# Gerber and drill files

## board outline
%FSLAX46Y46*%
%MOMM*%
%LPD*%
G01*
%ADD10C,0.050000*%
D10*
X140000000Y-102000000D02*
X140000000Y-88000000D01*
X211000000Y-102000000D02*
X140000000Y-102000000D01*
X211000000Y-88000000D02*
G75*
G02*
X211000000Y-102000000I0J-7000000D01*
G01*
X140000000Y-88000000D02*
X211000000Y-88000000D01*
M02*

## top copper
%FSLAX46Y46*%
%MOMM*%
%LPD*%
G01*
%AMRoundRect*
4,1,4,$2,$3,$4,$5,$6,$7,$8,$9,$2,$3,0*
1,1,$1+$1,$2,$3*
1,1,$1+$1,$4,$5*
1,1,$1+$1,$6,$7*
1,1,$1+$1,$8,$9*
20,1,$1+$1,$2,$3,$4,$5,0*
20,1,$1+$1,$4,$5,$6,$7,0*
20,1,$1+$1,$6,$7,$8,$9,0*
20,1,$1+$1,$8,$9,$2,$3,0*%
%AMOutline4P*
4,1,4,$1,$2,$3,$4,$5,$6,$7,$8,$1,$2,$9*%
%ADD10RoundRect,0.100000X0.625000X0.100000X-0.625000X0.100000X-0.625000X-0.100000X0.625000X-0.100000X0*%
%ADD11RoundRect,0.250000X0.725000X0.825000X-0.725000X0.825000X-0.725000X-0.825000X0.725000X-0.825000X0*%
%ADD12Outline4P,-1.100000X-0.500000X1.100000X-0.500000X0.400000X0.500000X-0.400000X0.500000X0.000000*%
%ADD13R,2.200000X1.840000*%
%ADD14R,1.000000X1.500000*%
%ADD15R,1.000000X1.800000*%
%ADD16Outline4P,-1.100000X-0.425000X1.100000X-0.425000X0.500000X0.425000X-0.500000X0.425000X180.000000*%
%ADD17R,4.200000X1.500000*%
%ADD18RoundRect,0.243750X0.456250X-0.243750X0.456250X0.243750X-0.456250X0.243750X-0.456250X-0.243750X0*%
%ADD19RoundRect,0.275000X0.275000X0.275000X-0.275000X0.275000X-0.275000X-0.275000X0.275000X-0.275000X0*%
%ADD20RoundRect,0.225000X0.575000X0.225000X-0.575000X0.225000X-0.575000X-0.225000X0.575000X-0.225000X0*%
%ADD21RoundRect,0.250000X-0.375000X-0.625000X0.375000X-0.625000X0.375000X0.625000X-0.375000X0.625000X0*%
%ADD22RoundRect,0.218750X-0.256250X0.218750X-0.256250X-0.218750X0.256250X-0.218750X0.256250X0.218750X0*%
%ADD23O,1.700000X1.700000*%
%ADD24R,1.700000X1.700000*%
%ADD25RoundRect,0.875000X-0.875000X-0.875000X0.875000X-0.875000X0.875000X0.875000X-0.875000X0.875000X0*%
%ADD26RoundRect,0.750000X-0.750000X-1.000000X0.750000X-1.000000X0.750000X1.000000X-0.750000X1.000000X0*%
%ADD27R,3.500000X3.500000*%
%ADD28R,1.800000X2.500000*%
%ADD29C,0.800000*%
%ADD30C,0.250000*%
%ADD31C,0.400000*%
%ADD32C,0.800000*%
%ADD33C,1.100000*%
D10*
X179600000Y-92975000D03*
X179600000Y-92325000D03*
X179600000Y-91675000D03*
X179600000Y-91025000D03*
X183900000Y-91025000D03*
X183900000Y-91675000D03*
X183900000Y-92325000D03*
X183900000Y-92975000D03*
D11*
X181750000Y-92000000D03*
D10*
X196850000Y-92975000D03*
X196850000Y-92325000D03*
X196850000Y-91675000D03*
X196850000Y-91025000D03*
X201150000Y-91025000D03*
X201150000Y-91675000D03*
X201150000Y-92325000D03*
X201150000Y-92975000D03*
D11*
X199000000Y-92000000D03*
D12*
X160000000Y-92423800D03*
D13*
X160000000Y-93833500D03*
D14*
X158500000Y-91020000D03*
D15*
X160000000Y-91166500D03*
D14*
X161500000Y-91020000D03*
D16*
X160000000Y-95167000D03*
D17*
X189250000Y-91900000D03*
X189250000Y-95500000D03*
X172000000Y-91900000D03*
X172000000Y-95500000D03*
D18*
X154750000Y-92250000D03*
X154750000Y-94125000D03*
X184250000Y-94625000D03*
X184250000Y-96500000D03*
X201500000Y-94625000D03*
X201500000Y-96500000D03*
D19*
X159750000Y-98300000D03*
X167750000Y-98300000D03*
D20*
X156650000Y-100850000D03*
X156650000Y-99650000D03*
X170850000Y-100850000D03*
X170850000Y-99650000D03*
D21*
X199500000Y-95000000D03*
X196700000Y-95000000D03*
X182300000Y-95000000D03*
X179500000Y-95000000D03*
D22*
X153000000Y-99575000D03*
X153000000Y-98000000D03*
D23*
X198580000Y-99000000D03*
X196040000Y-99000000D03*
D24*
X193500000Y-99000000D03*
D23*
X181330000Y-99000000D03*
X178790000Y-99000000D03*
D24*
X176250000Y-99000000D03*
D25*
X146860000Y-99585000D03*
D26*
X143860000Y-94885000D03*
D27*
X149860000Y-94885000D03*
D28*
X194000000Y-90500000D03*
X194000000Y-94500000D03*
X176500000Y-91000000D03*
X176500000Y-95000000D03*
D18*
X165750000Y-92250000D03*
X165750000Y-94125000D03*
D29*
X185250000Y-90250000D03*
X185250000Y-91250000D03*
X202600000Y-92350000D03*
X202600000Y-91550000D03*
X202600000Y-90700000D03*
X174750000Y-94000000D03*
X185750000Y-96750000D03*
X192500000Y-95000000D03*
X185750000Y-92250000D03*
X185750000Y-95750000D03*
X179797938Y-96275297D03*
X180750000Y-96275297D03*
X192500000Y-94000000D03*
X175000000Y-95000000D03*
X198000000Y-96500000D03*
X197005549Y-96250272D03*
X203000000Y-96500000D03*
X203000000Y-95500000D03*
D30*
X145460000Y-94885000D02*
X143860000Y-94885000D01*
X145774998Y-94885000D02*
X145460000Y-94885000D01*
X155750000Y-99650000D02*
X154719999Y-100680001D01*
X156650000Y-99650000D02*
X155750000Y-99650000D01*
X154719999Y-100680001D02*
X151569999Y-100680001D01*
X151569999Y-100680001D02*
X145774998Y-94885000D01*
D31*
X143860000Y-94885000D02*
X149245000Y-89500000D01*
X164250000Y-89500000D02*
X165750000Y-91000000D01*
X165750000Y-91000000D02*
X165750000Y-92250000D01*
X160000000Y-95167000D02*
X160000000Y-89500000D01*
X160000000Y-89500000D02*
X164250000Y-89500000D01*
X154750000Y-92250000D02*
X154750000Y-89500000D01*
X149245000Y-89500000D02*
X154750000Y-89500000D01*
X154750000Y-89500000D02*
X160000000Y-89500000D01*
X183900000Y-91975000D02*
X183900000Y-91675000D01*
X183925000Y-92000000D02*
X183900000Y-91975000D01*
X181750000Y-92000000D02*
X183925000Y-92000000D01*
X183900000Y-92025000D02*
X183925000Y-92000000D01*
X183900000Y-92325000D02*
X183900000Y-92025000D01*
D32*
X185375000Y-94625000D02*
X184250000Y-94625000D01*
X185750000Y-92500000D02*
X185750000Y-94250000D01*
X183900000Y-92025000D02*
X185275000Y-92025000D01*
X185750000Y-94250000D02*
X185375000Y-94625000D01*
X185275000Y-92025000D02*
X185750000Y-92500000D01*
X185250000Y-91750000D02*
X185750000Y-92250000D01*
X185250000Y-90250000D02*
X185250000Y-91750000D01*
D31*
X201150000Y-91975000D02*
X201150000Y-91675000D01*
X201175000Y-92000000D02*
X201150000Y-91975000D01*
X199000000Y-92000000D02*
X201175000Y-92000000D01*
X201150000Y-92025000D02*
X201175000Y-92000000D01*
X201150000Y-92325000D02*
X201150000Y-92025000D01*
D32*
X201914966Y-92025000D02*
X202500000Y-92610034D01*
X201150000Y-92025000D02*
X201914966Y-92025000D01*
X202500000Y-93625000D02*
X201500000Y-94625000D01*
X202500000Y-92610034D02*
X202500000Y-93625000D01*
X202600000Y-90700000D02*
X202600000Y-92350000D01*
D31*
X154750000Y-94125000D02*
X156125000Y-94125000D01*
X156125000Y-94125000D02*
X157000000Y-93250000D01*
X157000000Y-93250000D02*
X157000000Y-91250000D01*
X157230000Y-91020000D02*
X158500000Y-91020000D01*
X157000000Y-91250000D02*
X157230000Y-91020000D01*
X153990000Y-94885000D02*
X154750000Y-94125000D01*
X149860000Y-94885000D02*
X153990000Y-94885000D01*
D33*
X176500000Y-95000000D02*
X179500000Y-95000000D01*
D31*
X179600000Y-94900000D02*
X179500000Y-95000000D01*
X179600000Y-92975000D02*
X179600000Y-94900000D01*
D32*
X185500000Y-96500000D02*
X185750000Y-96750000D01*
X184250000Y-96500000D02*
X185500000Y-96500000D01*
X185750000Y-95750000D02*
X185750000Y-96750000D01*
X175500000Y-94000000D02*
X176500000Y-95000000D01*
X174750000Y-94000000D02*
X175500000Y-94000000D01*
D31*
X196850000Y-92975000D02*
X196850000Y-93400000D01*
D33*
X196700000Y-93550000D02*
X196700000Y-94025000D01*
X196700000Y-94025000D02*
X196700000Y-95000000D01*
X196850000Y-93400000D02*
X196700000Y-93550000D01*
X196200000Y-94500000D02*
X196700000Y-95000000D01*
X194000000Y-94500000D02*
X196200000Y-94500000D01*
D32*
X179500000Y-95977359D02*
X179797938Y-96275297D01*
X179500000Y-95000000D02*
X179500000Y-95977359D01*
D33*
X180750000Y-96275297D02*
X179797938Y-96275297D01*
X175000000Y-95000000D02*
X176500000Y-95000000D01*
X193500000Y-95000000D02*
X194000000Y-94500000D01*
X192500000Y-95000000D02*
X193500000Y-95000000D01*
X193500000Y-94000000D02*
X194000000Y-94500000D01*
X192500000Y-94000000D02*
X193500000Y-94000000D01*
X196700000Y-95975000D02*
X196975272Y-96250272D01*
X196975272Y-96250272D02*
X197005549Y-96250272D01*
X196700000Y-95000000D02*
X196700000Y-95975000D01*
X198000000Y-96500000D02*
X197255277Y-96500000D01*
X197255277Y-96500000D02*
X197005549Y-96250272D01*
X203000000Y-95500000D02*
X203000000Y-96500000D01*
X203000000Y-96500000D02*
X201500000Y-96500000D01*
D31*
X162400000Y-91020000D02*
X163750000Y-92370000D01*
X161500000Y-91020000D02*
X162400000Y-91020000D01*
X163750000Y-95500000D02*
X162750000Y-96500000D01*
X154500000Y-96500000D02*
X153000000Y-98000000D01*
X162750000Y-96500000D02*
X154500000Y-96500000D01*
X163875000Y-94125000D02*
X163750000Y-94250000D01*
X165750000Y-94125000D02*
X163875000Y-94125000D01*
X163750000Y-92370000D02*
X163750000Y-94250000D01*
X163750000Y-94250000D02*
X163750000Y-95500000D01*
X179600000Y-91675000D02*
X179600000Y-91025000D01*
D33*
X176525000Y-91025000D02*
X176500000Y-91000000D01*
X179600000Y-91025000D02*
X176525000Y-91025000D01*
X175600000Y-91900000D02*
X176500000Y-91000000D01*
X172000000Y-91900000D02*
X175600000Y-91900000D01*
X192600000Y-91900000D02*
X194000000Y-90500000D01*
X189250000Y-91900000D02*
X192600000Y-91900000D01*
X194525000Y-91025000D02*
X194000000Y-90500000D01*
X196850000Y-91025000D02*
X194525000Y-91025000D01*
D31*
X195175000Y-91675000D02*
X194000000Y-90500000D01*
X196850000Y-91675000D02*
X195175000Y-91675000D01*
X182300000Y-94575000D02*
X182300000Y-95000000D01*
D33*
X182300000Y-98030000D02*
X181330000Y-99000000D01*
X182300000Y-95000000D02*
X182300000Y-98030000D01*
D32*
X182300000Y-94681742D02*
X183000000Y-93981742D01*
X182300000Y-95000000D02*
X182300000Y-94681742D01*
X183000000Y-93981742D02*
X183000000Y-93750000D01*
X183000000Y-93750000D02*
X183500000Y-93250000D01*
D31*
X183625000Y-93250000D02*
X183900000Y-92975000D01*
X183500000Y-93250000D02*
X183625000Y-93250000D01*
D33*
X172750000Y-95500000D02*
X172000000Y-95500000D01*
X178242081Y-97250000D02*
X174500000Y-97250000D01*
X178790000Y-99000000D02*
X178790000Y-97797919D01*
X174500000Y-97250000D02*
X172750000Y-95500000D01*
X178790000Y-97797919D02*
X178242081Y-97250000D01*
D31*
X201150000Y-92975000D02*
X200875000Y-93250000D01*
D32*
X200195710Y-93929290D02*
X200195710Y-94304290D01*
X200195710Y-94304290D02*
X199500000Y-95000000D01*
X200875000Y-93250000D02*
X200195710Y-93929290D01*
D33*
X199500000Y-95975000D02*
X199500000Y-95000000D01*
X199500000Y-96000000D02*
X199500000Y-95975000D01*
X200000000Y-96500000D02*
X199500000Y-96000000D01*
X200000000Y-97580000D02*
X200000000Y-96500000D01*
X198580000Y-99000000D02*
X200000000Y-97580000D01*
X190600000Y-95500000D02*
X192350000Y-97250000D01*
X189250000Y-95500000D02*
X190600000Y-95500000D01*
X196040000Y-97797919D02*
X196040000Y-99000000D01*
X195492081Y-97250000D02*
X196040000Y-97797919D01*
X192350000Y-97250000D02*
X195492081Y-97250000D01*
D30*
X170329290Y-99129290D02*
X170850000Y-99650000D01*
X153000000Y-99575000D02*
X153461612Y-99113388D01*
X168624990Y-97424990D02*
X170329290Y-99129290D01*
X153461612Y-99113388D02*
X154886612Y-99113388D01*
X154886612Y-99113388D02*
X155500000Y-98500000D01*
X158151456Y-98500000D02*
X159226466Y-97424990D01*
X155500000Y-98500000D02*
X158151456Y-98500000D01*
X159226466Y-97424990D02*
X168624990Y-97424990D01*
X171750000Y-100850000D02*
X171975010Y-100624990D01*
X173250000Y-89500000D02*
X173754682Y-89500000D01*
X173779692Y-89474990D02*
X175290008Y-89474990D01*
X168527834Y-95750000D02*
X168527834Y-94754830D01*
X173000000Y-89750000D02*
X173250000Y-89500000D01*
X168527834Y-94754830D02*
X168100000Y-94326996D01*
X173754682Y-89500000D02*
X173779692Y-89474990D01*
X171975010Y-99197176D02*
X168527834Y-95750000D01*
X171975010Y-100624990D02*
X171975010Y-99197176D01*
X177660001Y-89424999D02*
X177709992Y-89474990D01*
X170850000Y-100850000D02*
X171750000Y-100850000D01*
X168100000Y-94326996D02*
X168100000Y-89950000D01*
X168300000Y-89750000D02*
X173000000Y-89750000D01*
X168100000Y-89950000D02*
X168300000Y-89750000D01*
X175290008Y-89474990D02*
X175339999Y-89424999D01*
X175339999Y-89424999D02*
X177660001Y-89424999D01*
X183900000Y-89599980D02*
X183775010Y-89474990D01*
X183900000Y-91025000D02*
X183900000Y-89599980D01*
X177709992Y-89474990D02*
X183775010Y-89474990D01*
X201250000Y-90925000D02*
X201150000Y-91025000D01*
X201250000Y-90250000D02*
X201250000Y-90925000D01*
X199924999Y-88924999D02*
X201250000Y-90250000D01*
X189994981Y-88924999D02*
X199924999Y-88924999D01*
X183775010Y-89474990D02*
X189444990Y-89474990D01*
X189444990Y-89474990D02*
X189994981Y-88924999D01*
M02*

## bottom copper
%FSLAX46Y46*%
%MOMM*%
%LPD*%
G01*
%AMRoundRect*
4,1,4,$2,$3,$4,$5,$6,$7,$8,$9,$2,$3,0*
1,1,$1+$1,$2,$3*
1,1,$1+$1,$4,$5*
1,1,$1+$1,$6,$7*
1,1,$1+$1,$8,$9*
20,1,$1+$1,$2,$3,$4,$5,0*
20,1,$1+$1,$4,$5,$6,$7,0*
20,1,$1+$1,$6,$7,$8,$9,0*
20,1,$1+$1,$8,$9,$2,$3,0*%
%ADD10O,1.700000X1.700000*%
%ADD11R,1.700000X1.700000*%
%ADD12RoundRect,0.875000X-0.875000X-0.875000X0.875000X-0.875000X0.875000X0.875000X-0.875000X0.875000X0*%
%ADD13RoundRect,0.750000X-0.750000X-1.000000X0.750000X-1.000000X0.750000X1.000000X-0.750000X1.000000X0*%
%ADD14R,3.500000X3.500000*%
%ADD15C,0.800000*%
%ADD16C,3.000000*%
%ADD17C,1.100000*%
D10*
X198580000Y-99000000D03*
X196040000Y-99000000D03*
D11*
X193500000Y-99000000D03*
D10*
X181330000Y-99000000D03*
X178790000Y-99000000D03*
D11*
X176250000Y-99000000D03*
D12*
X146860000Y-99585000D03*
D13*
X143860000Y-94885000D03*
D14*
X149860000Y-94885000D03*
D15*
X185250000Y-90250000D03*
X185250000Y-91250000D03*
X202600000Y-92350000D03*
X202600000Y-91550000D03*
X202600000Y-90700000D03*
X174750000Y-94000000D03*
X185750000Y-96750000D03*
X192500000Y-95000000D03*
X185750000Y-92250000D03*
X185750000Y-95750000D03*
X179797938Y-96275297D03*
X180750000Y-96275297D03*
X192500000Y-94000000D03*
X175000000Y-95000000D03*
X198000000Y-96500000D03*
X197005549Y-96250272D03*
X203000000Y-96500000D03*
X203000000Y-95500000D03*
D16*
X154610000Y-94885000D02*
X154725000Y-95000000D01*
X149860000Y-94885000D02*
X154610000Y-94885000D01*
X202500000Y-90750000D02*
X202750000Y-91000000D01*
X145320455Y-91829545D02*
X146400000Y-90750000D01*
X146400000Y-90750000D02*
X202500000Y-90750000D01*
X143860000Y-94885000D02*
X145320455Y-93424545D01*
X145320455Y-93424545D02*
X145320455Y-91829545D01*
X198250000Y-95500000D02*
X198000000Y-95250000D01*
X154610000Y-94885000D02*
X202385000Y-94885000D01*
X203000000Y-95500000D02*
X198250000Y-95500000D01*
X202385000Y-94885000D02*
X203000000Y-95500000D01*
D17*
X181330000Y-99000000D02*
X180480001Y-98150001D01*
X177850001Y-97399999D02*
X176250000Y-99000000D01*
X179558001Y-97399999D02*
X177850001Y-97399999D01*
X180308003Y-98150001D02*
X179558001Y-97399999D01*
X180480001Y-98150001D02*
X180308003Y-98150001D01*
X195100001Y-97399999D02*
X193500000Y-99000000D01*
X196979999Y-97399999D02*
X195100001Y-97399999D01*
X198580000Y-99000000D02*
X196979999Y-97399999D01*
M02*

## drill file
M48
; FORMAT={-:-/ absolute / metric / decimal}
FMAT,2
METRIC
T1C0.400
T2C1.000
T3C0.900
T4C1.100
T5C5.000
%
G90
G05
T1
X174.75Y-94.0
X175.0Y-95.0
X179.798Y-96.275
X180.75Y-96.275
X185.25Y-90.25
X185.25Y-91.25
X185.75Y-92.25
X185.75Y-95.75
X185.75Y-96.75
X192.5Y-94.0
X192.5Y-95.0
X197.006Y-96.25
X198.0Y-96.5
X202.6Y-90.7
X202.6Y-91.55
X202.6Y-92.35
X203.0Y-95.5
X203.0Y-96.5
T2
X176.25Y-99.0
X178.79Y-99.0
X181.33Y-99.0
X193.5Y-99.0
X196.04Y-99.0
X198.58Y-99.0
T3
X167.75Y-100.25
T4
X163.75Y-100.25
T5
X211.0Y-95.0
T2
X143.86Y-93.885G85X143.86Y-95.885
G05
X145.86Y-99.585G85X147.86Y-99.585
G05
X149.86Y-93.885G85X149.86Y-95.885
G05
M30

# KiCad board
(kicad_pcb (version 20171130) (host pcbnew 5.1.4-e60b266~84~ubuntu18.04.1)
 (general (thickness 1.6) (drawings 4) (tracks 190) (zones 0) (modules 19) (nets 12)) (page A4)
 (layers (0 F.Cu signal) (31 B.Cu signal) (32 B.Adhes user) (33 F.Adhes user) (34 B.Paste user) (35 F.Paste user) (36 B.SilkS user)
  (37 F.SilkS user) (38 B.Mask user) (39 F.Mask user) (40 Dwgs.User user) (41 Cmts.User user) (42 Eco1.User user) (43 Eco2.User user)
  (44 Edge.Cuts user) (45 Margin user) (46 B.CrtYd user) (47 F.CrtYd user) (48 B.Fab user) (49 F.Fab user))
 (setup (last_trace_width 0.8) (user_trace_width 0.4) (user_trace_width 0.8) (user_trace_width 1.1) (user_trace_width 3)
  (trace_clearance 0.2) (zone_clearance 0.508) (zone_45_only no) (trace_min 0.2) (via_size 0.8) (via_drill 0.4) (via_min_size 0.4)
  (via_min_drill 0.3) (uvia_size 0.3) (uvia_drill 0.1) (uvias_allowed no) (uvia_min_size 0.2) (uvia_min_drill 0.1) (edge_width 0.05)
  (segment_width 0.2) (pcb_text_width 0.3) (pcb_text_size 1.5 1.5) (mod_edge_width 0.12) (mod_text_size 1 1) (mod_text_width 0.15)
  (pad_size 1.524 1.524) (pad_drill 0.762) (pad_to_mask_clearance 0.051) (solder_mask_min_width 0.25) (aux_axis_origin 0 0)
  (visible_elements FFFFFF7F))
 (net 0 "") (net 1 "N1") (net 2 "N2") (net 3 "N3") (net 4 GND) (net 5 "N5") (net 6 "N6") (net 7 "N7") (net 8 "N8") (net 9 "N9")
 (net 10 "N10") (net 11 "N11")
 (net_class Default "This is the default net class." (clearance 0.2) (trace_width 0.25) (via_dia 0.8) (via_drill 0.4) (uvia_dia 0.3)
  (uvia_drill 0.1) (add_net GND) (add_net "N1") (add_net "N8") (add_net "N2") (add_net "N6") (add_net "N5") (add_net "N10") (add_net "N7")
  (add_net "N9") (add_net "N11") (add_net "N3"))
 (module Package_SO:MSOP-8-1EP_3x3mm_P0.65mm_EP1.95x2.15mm (layer F.Cu) (at 181.75 92 180)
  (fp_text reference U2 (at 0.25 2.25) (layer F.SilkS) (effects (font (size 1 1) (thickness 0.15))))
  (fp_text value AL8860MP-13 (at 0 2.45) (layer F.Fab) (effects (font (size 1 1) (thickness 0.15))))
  (pad 8 smd roundrect (at 2.15 -0.975 180) (size 1.45 0.4) (layers F.Cu F.Paste F.Mask) (roundrect_rratio 0.25) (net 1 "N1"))
  (pad 7 smd roundrect (at 2.15 -0.325 180) (size 1.45 0.4) (layers F.Cu F.Paste F.Mask) (roundrect_rratio 0.25))
  (pad 6 smd roundrect (at 2.15 0.325 180) (size 1.45 0.4) (layers F.Cu F.Paste F.Mask) (roundrect_rratio 0.25) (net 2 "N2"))
  (pad 5 smd roundrect (at 2.15 0.975 180) (size 1.45 0.4) (layers F.Cu F.Paste F.Mask) (roundrect_rratio 0.25) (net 2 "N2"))
  (pad 4 smd roundrect (at -2.15 0.975 180) (size 1.45 0.4) (layers F.Cu F.Paste F.Mask) (roundrect_rratio 0.25) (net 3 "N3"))
  (pad 3 smd roundrect (at -2.15 0.325 180) (size 1.45 0.4) (layers F.Cu F.Paste F.Mask) (roundrect_rratio 0.25) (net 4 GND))
  (pad 2 smd roundrect (at -2.15 -0.325 180) (size 1.45 0.4) (layers F.Cu F.Paste F.Mask) (roundrect_rratio 0.25) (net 4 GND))
  (pad 1 smd roundrect (at -2.15 -0.975 180) (size 1.45 0.4) (layers F.Cu F.Paste F.Mask) (roundrect_rratio 0.25) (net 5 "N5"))
  (pad "" smd roundrect (at 0.49 0.54 180) (size 0.79 0.87) (layers F.Paste) (roundrect_rratio 0.25))
  (pad "" smd roundrect (at 0.49 -0.54 180) (size 0.79 0.87) (layers F.Paste) (roundrect_rratio 0.25))
  (pad "" smd roundrect (at -0.49 0.54 180) (size 0.79 0.87) (layers F.Paste) (roundrect_rratio 0.25))
  (pad "" smd roundrect (at -0.49 -0.54 180) (size 0.79 0.87) (layers F.Paste) (roundrect_rratio 0.25))
  (pad 9 smd roundrect (at 0 0 180) (size 1.95 2.15) (layers F.Cu F.Mask) (roundrect_rratio 0.128205) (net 4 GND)))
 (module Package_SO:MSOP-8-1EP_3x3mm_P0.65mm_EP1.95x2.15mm (layer F.Cu) (at 199 92 180)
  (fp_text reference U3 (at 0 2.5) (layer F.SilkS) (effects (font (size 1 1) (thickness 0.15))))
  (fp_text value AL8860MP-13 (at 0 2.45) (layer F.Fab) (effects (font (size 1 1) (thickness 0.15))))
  (pad 8 smd roundrect (at 2.15 -0.975 180) (size 1.45 0.4) (layers F.Cu F.Paste F.Mask) (roundrect_rratio 0.25) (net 1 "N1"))
  (pad 7 smd roundrect (at 2.15 -0.325 180) (size 1.45 0.4) (layers F.Cu F.Paste F.Mask) (roundrect_rratio 0.25))
  (pad 6 smd roundrect (at 2.15 0.325 180) (size 1.45 0.4) (layers F.Cu F.Paste F.Mask) (roundrect_rratio 0.25) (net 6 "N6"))
  (pad 5 smd roundrect (at 2.15 0.975 180) (size 1.45 0.4) (layers F.Cu F.Paste F.Mask) (roundrect_rratio 0.25) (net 6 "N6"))
  (pad 4 smd roundrect (at -2.15 0.975 180) (size 1.45 0.4) (layers F.Cu F.Paste F.Mask) (roundrect_rratio 0.25) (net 3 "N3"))
  (pad 3 smd roundrect (at -2.15 0.325 180) (size 1.45 0.4) (layers F.Cu F.Paste F.Mask) (roundrect_rratio 0.25) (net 4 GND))
  (pad 2 smd roundrect (at -2.15 -0.325 180) (size 1.45 0.4) (layers F.Cu F.Paste F.Mask) (roundrect_rratio 0.25) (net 4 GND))
  (pad 1 smd roundrect (at -2.15 -0.975 180) (size 1.45 0.4) (layers F.Cu F.Paste F.Mask) (roundrect_rratio 0.25) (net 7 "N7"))
  (pad "" smd roundrect (at 0.49 0.54 180) (size 0.79 0.87) (layers F.Paste) (roundrect_rratio 0.25))
  (pad "" smd roundrect (at 0.49 -0.54 180) (size 0.79 0.87) (layers F.Paste) (roundrect_rratio 0.25))
  (pad "" smd roundrect (at -0.49 0.54 180) (size 0.79 0.87) (layers F.Paste) (roundrect_rratio 0.25))
  (pad "" smd roundrect (at -0.49 -0.54 180) (size 0.79 0.87) (layers F.Paste) (roundrect_rratio 0.25))
  (pad 9 smd roundrect (at 0 0 180) (size 1.95 2.15) (layers F.Cu F.Mask) (roundrect_rratio 0.128205) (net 4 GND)))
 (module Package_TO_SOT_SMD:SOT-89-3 (layer F.Cu) (at 160 92.5 270)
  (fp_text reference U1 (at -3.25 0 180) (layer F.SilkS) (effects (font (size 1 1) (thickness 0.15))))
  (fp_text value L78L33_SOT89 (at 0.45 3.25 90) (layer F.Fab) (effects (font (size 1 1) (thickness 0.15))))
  (pad 2 smd trapezoid (at -0.0762 0) (size 1.5 1) (rect_delta 0 0.7) (layers F.Cu F.Paste F.Mask) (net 4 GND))
  (pad 2 smd rect (at 1.3335 0 180) (size 2.2 1.84) (layers F.Cu F.Paste F.Mask) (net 4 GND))
  (pad 3 smd rect (at -1.48 1.5 180) (size 1 1.5) (layers F.Cu F.Paste F.Mask) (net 1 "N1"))
  (pad 2 smd rect (at -1.3335 0 180) (size 1 1.8) (layers F.Cu F.Paste F.Mask) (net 4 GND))
  (pad 1 smd rect (at -1.48 -1.5 180) (size 1 1.5) (layers F.Cu F.Paste F.Mask) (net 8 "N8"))
  (pad 2 smd trapezoid (at 2.667 0 180) (size 1.6 0.85) (rect_delta 0 0.6) (layers F.Cu F.Paste F.Mask) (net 4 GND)))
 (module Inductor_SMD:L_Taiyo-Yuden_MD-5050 (layer F.Cu) (at 189.25 93.7 90)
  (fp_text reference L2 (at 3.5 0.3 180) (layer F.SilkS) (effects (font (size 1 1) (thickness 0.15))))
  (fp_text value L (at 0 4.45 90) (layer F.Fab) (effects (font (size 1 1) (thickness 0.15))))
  (pad 2 smd rect (at 1.8 0 90) (size 1.5 4.2) (layers F.Cu F.Paste F.Mask) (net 6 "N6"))
  (pad 1 smd rect (at -1.8 0 90) (size 1.5 4.2) (layers F.Cu F.Paste F.Mask) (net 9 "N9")))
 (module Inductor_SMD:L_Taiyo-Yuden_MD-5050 (layer F.Cu) (at 172 93.7 90)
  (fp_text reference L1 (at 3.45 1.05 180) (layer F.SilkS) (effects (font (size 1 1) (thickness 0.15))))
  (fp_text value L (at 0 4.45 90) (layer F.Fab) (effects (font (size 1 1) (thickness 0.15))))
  (pad 2 smd rect (at 1.8 0 90) (size 1.5 4.2) (layers F.Cu F.Paste F.Mask) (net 2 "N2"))
  (pad 1 smd rect (at -1.8 0 90) (size 1.5 4.2) (layers F.Cu F.Paste F.Mask) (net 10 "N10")))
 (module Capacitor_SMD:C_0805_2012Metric (layer F.Cu) (at 154.75 93.1875 90)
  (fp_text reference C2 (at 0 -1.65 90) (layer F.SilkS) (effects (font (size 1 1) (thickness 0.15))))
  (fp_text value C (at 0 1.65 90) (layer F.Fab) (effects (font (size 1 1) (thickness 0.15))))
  (pad 2 smd roundrect (at 0.9375 0 90) (size 0.975 1.4) (layers F.Cu F.Paste F.Mask) (roundrect_rratio 0.25) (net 4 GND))
  (pad 1 smd roundrect (at -0.9375 0 90) (size 0.975 1.4) (layers F.Cu F.Paste F.Mask) (roundrect_rratio 0.25) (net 1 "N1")))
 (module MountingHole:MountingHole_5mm (layer F.Cu) (at 211 95)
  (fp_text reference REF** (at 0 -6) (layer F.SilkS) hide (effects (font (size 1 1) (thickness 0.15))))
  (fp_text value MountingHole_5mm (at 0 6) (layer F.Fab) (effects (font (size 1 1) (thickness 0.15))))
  (pad 1 np_thru_hole circle (at 0 0) (size 5 5) (drill 5) (layers *.Cu *.Mask)))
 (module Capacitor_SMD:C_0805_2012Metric (layer F.Cu) (at 184.25 95.5625 90)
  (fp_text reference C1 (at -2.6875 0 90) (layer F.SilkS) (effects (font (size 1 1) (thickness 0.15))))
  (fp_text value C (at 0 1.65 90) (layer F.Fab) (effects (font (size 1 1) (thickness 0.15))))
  (pad 2 smd roundrect (at 0.9375 0 90) (size 0.975 1.4) (layers F.Cu F.Paste F.Mask) (roundrect_rratio 0.25) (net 4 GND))
  (pad 1 smd roundrect (at -0.9375 0 90) (size 0.975 1.4) (layers F.Cu F.Paste F.Mask) (roundrect_rratio 0.25) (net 1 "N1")))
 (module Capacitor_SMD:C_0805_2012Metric (layer F.Cu) (at 201.5 95.5625 90)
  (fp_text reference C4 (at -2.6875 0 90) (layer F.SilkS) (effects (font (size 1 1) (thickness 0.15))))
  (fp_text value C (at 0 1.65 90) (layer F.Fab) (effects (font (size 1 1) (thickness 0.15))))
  (pad 2 smd roundrect (at 0.9375 0 90) (size 0.975 1.4) (layers F.Cu F.Paste F.Mask) (roundrect_rratio 0.25) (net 4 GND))
  (pad 1 smd roundrect (at -0.9375 0 90) (size 0.975 1.4) (layers F.Cu F.Paste F.Mask) (roundrect_rratio 0.25) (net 1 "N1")))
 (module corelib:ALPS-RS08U (layer F.Cu) (at 163.75 100.25 180)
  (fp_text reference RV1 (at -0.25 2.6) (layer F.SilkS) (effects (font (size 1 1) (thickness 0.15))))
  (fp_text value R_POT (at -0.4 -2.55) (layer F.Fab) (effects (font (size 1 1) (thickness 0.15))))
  (pad "" smd roundrect (at 4 1.95 180) (size 1.1 1.1) (layers F.Cu F.Paste F.Mask) (roundrect_rratio 0.25))
  (pad "" smd roundrect (at -4 1.95 180) (size 1.1 1.1) (layers F.Cu F.Paste F.Mask) (roundrect_rratio 0.25))
  (pad "" smd roundrect (at 7.1 -0.6 180) (size 1.6 0.9) (layers F.Cu F.Paste F.Mask) (roundrect_rratio 0.25))
  (pad 3 smd roundrect (at 7.1 0.6 180) (size 1.6 0.9) (layers F.Cu F.Paste F.Mask) (roundrect_rratio 0.25) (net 4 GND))
  (pad 2 smd roundrect (at -7.1 -0.6 180) (size 1.6 0.9) (layers F.Cu F.Paste F.Mask) (roundrect_rratio 0.25) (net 3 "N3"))
  (pad 1 smd roundrect (at -7.1 0.6 180) (size 1.6 0.9) (layers F.Cu F.Paste F.Mask) (roundrect_rratio 0.25) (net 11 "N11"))
  (pad "" np_thru_hole circle (at -4 0 180) (size 0.9 0.9) (drill 0.9) (layers *.Cu *.Mask))
  (pad "" np_thru_hole circle (at 0 0 180) (size 1.1 1.1) (drill 1.1) (layers *.Cu *.Mask)))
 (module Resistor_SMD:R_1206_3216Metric (layer F.Cu) (at 198.1 95)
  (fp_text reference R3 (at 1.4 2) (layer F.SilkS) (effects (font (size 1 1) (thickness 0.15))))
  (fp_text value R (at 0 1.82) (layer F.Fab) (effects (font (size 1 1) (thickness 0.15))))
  (pad 2 smd roundrect (at 1.4 0) (size 1.25 1.75) (layers F.Cu F.Paste F.Mask) (roundrect_rratio 0.2) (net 7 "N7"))
  (pad 1 smd roundrect (at -1.4 0) (size 1.25 1.75) (layers F.Cu F.Paste F.Mask) (roundrect_rratio 0.2) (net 1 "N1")))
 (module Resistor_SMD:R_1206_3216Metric (layer F.Cu) (at 180.9 95)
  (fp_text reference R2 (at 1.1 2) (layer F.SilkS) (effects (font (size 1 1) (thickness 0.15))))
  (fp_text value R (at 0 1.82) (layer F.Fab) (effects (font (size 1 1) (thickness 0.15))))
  (pad 2 smd roundrect (at 1.4 0) (size 1.25 1.75) (layers F.Cu F.Paste F.Mask) (roundrect_rratio 0.2) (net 5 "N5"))
  (pad 1 smd roundrect (at -1.4 0) (size 1.25 1.75) (layers F.Cu F.Paste F.Mask) (roundrect_rratio 0.2) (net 1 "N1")))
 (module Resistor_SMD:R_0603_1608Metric (layer F.Cu) (at 153 98.7875 270)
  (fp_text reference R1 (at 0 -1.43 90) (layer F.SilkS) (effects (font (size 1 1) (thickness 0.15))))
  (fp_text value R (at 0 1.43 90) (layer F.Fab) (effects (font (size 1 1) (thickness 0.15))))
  (pad 2 smd roundrect (at 0.7875 0 270) (size 0.875 0.95) (layers F.Cu F.Paste F.Mask) (roundrect_rratio 0.25) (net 11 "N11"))
  (pad 1 smd roundrect (at -0.7875 0 270) (size 0.875 0.95) (layers F.Cu F.Paste F.Mask) (roundrect_rratio 0.25) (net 8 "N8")))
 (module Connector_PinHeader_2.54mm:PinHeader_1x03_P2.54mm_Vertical (layer F.Cu) (at 193.5 99 90)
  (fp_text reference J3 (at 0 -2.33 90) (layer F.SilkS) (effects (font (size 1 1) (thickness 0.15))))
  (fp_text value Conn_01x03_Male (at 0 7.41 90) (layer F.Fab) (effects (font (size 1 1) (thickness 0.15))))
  (pad 3 thru_hole oval (at 0 5.08 90) (size 1.7 1.7) (drill 1) (layers *.Cu *.Mask) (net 7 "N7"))
  (pad 2 thru_hole oval (at 0 2.54 90) (size 1.7 1.7) (drill 1) (layers *.Cu *.Mask) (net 9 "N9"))
  (pad 1 thru_hole rect (at 0 0 90) (size 1.7 1.7) (drill 1) (layers *.Cu *.Mask) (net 7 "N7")))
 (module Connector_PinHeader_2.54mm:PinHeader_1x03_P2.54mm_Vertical (layer F.Cu) (at 176.25 99 90)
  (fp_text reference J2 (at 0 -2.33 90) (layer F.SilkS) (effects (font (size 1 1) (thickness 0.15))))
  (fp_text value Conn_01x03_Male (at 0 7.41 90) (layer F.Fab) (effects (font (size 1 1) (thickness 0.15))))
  (pad 3 thru_hole oval (at 0 5.08 90) (size 1.7 1.7) (drill 1) (layers *.Cu *.Mask) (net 5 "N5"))
  (pad 2 thru_hole oval (at 0 2.54 90) (size 1.7 1.7) (drill 1) (layers *.Cu *.Mask) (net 10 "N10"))
  (pad 1 thru_hole rect (at 0 0 90) (size 1.7 1.7) (drill 1) (layers *.Cu *.Mask) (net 5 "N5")))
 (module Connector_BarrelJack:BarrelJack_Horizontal (layer F.Cu) (at 149.86 94.885)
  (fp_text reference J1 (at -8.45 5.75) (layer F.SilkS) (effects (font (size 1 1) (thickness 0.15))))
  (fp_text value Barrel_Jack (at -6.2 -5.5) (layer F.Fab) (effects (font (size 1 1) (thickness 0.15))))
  (pad 3 thru_hole roundrect (at -3 4.7) (size 3.5 3.5) (drill oval 3 1) (layers *.Cu *.Mask) (roundrect_rratio 0.25))
  (pad 2 thru_hole roundrect (at -6 0) (size 3 3.5) (drill oval 1 3) (layers *.Cu *.Mask) (roundrect_rratio 0.25) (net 4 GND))
  (pad 1 thru_hole rect (at 0 0) (size 3.5 3.5) (drill oval 1 3) (layers *.Cu *.Mask) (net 1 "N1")))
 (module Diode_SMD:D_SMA (layer F.Cu) (at 194 92.5 90)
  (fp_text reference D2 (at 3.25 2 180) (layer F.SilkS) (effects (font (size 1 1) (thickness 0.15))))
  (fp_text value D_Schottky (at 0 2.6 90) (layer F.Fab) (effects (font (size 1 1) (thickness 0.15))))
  (pad 2 smd rect (at 2 0 90) (size 2.5 1.8) (layers F.Cu F.Paste F.Mask) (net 6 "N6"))
  (pad 1 smd rect (at -2 0 90) (size 2.5 1.8) (layers F.Cu F.Paste F.Mask) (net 1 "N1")))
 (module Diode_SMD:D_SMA (layer F.Cu) (at 176.5 93 90)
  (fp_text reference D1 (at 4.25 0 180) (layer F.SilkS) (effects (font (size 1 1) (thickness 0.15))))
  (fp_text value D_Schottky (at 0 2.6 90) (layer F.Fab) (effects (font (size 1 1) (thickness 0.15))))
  (pad 2 smd rect (at 2 0 90) (size 2.5 1.8) (layers F.Cu F.Paste F.Mask) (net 2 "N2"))
  (pad 1 smd rect (at -2 0 90) (size 2.5 1.8) (layers F.Cu F.Paste F.Mask) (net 1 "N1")))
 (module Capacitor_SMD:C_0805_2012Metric (layer F.Cu) (at 165.75 93.1875 90)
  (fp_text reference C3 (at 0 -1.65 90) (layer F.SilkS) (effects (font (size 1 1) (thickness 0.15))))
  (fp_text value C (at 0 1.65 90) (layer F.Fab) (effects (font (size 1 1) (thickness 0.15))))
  (pad 2 smd roundrect (at 0.9375 0 90) (size 0.975 1.4) (layers F.Cu F.Paste F.Mask) (roundrect_rratio 0.25) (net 4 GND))
  (pad 1 smd roundrect (at -0.9375 0 90) (size 0.975 1.4) (layers F.Cu F.Paste F.Mask) (roundrect_rratio 0.25) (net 8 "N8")))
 (gr_line (start 140 102) (end 140 88) (layer Edge.Cuts) (width 0.05))
 (gr_line (start 211 102) (end 140 102) (layer Edge.Cuts) (width 0.05))
 (gr_arc (start 211 95) (end 211 102) (angle -180) (layer Edge.Cuts) (width 0.05))
 (gr_line (start 140 88) (end 211 88) (layer Edge.Cuts) (width 0.05))
 (via (at 185.25 90.25) (size 0.8) (drill 0.4) (layers F.Cu B.Cu) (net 4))
 (via (at 185.25 91.25) (size 0.8) (drill 0.4) (layers F.Cu B.Cu) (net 4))
 (via (at 202.6 92.35) (size 0.8) (drill 0.4) (layers F.Cu B.Cu) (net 4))
 (via (at 202.6 91.55) (size 0.8) (drill 0.4) (layers F.Cu B.Cu) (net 4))
 (via (at 202.6 90.7) (size 0.8) (drill 0.4) (layers F.Cu B.Cu) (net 4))
 (segment (start 154.61 94.885) (end 154.725 95) (width 3) (layer B.Cu) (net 1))
 (segment (start 149.86 94.885) (end 154.61 94.885) (width 3) (layer B.Cu) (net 1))
 (via (at 174.75 94) (size 0.8) (drill 0.4) (layers F.Cu B.Cu) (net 1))
 (via (at 185.75 96.75) (size 0.8) (drill 0.4) (layers F.Cu B.Cu) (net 1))
 (via (at 192.5 95) (size 0.8) (drill 0.4) (layers F.Cu B.Cu) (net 1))
 (segment (start 145.46 94.885) (end 143.86 94.885) (width 0.25) (layer F.Cu) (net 4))
 (segment (start 145.774998 94.885) (end 145.46 94.885) (width 0.25) (layer F.Cu) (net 4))
 (segment (start 155.75 99.65) (end 154.719999 100.680001) (width 0.25) (layer F.Cu) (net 4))
 (segment (start 156.65 99.65) (end 155.75 99.65) (width 0.25) (layer F.Cu) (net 4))
 (segment (start 154.719999 100.680001) (end 151.569999 100.680001) (width 0.25) (layer F.Cu) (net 4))
 (segment (start 151.569999 100.680001) (end 145.774998 94.885) (width 0.25) (layer F.Cu) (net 4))
 (via (at 185.75 92.25) (size 0.8) (drill 0.4) (layers F.Cu B.Cu) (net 4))
 (segment (start 143.86 94.885) (end 149.245 89.5) (width 0.4) (layer F.Cu) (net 4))
 (segment (start 164.25 89.5) (end 165.75 91) (width 0.4) (layer F.Cu) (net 4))
 (segment (start 165.75 91) (end 165.75 92.25) (width 0.4) (layer F.Cu) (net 4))
 (segment (start 160 95.167) (end 160 89.5) (width 0.4) (layer F.Cu) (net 4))
 (segment (start 160 89.5) (end 164.25 89.5) (width 0.4) (layer F.Cu) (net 4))
 (segment (start 154.75 92.25) (end 154.75 89.5) (width 0.4) (layer F.Cu) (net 4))
 (segment (start 149.245 89.5) (end 154.75 89.5) (width 0.4) (layer F.Cu) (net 4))
 (segment (start 154.75 89.5) (end 160 89.5) (width 0.4) (layer F.Cu) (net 4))
 (segment (start 183.9 91.975) (end 183.9 91.675) (width 0.4) (layer F.Cu) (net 4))
 (segment (start 183.925 92) (end 183.9 91.975) (width 0.4) (layer F.Cu) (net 4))
 (segment (start 181.75 92) (end 183.925 92) (width 0.4) (layer F.Cu) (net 4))
 (segment (start 183.9 92.025) (end 183.925 92) (width 0.4) (layer F.Cu) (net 4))
 (segment (start 183.9 92.325) (end 183.9 92.025) (width 0.4) (layer F.Cu) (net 4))
 (segment (start 185.375 94.625) (end 184.25 94.625) (width 0.8) (layer F.Cu) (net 4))
 (segment (start 185.75 92.5) (end 185.75 94.25) (width 0.8) (layer F.Cu) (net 4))
 (segment (start 183.9 92.025) (end 185.275 92.025) (width 0.8) (layer F.Cu) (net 4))
 (segment (start 185.75 94.25) (end 185.375 94.625) (width 0.8) (layer F.Cu) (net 4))
 (segment (start 185.275 92.025) (end 185.75 92.5) (width 0.8) (layer F.Cu) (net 4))
 (segment (start 185.25 91.75) (end 185.75 92.25) (width 0.8) (layer F.Cu) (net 4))
 (segment (start 185.25 90.25) (end 185.25 91.75) (width 0.8) (layer F.Cu) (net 4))
 (segment (start 201.15 91.975) (end 201.15 91.675) (width 0.4) (layer F.Cu) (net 4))
 (segment (start 201.175 92) (end 201.15 91.975) (width 0.4) (layer F.Cu) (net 4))
 (segment (start 199 92) (end 201.175 92) (width 0.4) (layer F.Cu) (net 4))
 (segment (start 201.15 92.025) (end 201.175 92) (width 0.4) (layer F.Cu) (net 4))
 (segment (start 201.15 92.325) (end 201.15 92.025) (width 0.4) (layer F.Cu) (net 4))
 (segment (start 201.914966 92.025) (end 202.5 92.610034) (width 0.8) (layer F.Cu) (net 4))
 (segment (start 201.15 92.025) (end 201.914966 92.025) (width 0.8) (layer F.Cu) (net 4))
 (segment (start 202.5 93.625) (end 201.5 94.625) (width 0.8) (layer F.Cu) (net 4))
 (segment (start 202.5 92.610034) (end 202.5 93.625) (width 0.8) (layer F.Cu) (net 4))
 (segment (start 202.5 90.75) (end 202.75 91) (width 3) (layer B.Cu) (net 4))
 (segment (start 145.320455 91.829545) (end 146.4 90.75) (width 3) (layer B.Cu) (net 4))
 (segment (start 146.4 90.75) (end 202.5 90.75) (width 3) (layer B.Cu) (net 4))
 (segment (start 143.86 94.885) (end 145.320455 93.424545) (width 3) (layer B.Cu) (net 4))
 (segment (start 145.320455 93.424545) (end 145.320455 91.829545) (width 3) (layer B.Cu) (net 4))
 (segment (start 202.6 90.7) (end 202.6 92.35) (width 0.8) (layer F.Cu) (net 4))
 (segment (start 154.75 94.125) (end 156.125 94.125) (width 0.4) (layer F.Cu) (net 1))
 (segment (start 156.125 94.125) (end 157 93.25) (width 0.4) (layer F.Cu) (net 1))
 (segment (start 157 93.25) (end 157 91.25) (width 0.4) (layer F.Cu) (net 1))
 (segment (start 157.23 91.02) (end 158.5 91.02) (width 0.4) (layer F.Cu) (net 1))
 (segment (start 157 91.25) (end 157.23 91.02) (width 0.4) (layer F.Cu) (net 1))
 (segment (start 153.99 94.885) (end 154.75 94.125) (width 0.4) (layer F.Cu) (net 1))
 (segment (start 149.86 94.885) (end 153.99 94.885) (width 0.4) (layer F.Cu) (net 1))
 (segment (start 176.5 95) (end 179.5 95) (width 1.1) (layer F.Cu) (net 1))
 (segment (start 179.6 94.9) (end 179.5 95) (width 0.4) (layer F.Cu) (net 1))
 (segment (start 179.6 92.975) (end 179.6 94.9) (width 0.4) (layer F.Cu) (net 1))
 (via (at 185.75 95.75) (size 0.8) (drill 0.4) (layers F.Cu B.Cu) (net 1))
 (segment (start 185.5 96.5) (end 185.75 96.75) (width 0.8) (layer F.Cu) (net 1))
 (segment (start 184.25 96.5) (end 185.5 96.5) (width 0.8) (layer F.Cu) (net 1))
 (segment (start 185.75 95.75) (end 185.75 96.75) (width 0.8) (layer F.Cu) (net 1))
 (segment (start 175.5 94) (end 176.5 95) (width 0.8) (layer F.Cu) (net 1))
 (segment (start 174.75 94) (end 175.5 94) (width 0.8) (layer F.Cu) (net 1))
 (segment (start 196.85 92.975) (end 196.85 93.4) (width 0.4) (layer F.Cu) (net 1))
 (segment (start 196.7 93.55) (end 196.7 94.025) (width 1.1) (layer F.Cu) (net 1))
 (segment (start 196.7 94.025) (end 196.7 95) (width 1.1) (layer F.Cu) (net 1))
 (segment (start 196.85 93.4) (end 196.7 93.55) (width 1.1) (layer F.Cu) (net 1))
 (segment (start 196.2 94.5) (end 196.7 95) (width 1.1) (layer F.Cu) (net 1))
 (segment (start 194 94.5) (end 196.2 94.5) (width 1.1) (layer F.Cu) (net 1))
 (via (at 179.797938 96.275297) (size 0.8) (drill 0.4) (layers F.Cu B.Cu) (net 1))
 (segment (start 179.5 95.977359) (end 179.797938 96.275297) (width 0.8) (layer F.Cu) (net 1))
 (segment (start 179.5 95) (end 179.5 95.977359) (width 0.8) (layer F.Cu) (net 1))
 (via (at 180.75 96.275297) (size 0.8) (drill 0.4) (layers F.Cu B.Cu) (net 1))
 (segment (start 180.75 96.275297) (end 179.797938 96.275297) (width 1.1) (layer F.Cu) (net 1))
 (via (at 192.5 94) (size 0.8) (drill 0.4) (layers F.Cu B.Cu) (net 1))
 (via (at 175 95) (size 0.8) (drill 0.4) (layers F.Cu B.Cu) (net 1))
 (segment (start 175 95) (end 176.5 95) (width 1.1) (layer F.Cu) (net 1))
 (segment (start 193.5 95) (end 194 94.5) (width 1.1) (layer F.Cu) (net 1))
 (segment (start 192.5 95) (end 193.5 95) (width 1.1) (layer F.Cu) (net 1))
 (segment (start 193.5 94) (end 194 94.5) (width 1.1) (layer F.Cu) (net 1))
 (segment (start 192.5 94) (end 193.5 94) (width 1.1) (layer F.Cu) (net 1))
 (via (at 198 96.5) (size 0.8) (drill 0.4) (layers F.Cu B.Cu) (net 1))
 (segment (start 196.7 95.975) (end 196.975272 96.250272) (width 1.1) (layer F.Cu) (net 1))
 (segment (start 196.975272 96.250272) (end 197.005549 96.250272) (width 1.1) (layer F.Cu) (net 1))
 (segment (start 196.7 95) (end 196.7 95.975) (width 1.1) (layer F.Cu) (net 1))
 (segment (start 198 96.5) (end 197.255277 96.5) (width 1.1) (layer F.Cu) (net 1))
 (segment (start 197.255277 96.5) (end 197.005549 96.250272) (width 1.1) (layer F.Cu) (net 1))
 (via (at 197.005549 96.250272) (size 0.8) (drill 0.4) (layers F.Cu B.Cu) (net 1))
 (via (at 203 96.5) (size 0.8) (drill 0.4) (layers F.Cu B.Cu) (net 1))
 (via (at 203 95.5) (size 0.8) (drill 0.4) (layers F.Cu B.Cu) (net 1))
 (segment (start 203 95.5) (end 203 96.5) (width 1.1) (layer F.Cu) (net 1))
 (segment (start 203 96.5) (end 201.5 96.5) (width 1.1) (layer F.Cu) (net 1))
 (segment (start 198.25 95.5) (end 198 95.25) (width 3) (layer B.Cu) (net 1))
 (segment (start 154.61 94.885) (end 202.385 94.885) (width 3) (layer B.Cu) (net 1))
 (segment (start 203 95.5) (end 198.25 95.5) (width 3) (layer B.Cu) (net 1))
 (segment (start 202.385 94.885) (end 203 95.5) (width 3) (layer B.Cu) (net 1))
 (segment (start 162.4 91.02) (end 163.75 92.37) (width 0.4) (layer F.Cu) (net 8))
 (segment (start 161.5 91.02) (end 162.4 91.02) (width 0.4) (layer F.Cu) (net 8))
 (segment (start 163.75 95.5) (end 162.75 96.5) (width 0.4) (layer F.Cu) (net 8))
 (segment (start 154.5 96.5) (end 153 98) (width 0.4) (layer F.Cu) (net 8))
 (segment (start 162.75 96.5) (end 154.5 96.5) (width 0.4) (layer F.Cu) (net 8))
 (segment (start 163.875 94.125) (end 163.75 94.25) (width 0.4) (layer F.Cu) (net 8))
 (segment (start 165.75 94.125) (end 163.875 94.125) (width 0.4) (layer F.Cu) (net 8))
 (segment (start 163.75 92.37) (end 163.75 94.25) (width 0.4) (layer F.Cu) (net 8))
 (segment (start 163.75 94.25) (end 163.75 95.5) (width 0.4) (layer F.Cu) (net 8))
 (segment (start 179.6 91.675) (end 179.6 91.025) (width 0.4) (layer F.Cu) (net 2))
 (segment (start 176.525 91.025) (end 176.5 91) (width 1.1) (layer F.Cu) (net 2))
 (segment (start 179.6 91.025) (end 176.525 91.025) (width 1.1) (layer F.Cu) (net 2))
 (segment (start 175.6 91.9) (end 176.5 91) (width 1.1) (layer F.Cu) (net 2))
 (segment (start 172 91.9) (end 175.6 91.9) (width 1.1) (layer F.Cu) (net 2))
 (segment (start 192.6 91.9) (end 194 90.5) (width 1.1) (layer F.Cu) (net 6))
 (segment (start 189.25 91.9) (end 192.6 91.9) (width 1.1) (layer F.Cu) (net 6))
 (segment (start 194.525 91.025) (end 194 90.5) (width 1.1) (layer F.Cu) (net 6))
 (segment (start 196.85 91.025) (end 194.525 91.025) (width 1.1) (layer F.Cu) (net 6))
 (segment (start 195.175 91.675) (end 194 90.5) (width 0.4) (layer F.Cu) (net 6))
 (segment (start 196.85 91.675) (end 195.175 91.675) (width 0.4) (layer F.Cu) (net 6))
 (segment (start 182.3 94.575) (end 182.3 95) (width 0.4) (layer F.Cu) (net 5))
 (segment (start 182.3 98.03) (end 181.33 99) (width 1.1) (layer F.Cu) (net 5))
 (segment (start 182.3 95) (end 182.3 98.03) (width 1.1) (layer F.Cu) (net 5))
 (segment (start 182.3 94.681742) (end 183 93.981742) (width 0.8) (layer F.Cu) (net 5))
 (segment (start 182.3 95) (end 182.3 94.681742) (width 0.8) (layer F.Cu) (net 5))
 (segment (start 183 93.981742) (end 183 93.75) (width 0.8) (layer F.Cu) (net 5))
 (segment (start 183 93.75) (end 183.5 93.25) (width 0.8) (layer F.Cu) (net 5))
 (segment (start 183.625 93.25) (end 183.9 92.975) (width 0.4) (layer F.Cu) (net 5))
 (segment (start 183.5 93.25) (end 183.625 93.25) (width 0.4) (layer F.Cu) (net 5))
 (segment (start 181.33 99) (end 180.480001 98.150001) (width 1.1) (layer B.Cu) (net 5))
 (segment (start 177.850001 97.399999) (end 176.25 99) (width 1.1) (layer B.Cu) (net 5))
 (segment (start 179.558001 97.399999) (end 177.850001 97.399999) (width 1.1) (layer B.Cu) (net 5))
 (segment (start 180.308003 98.150001) (end 179.558001 97.399999) (width 1.1) (layer B.Cu) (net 5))
 (segment (start 180.480001 98.150001) (end 180.308003 98.150001) (width 1.1) (layer B.Cu) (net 5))
 (segment (start 172.75 95.5) (end 172 95.5) (width 1.1) (layer F.Cu) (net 10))
 (segment (start 178.242081 97.25) (end 174.5 97.25) (width 1.1) (layer F.Cu) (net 10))
 (segment (start 178.79 99) (end 178.79 97.797919) (width 1.1) (layer F.Cu) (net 10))
 (segment (start 174.5 97.25) (end 172.75 95.5) (width 1.1) (layer F.Cu) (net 10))
 (segment (start 178.79 97.797919) (end 178.242081 97.25) (width 1.1) (layer F.Cu) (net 10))
 (segment (start 201.15 92.975) (end 200.875 93.25) (width 0.4) (layer F.Cu) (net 7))
 (segment (start 200.19571 93.92929) (end 200.19571 94.30429) (width 0.8) (layer F.Cu) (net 7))
 (segment (start 200.19571 94.30429) (end 199.5 95) (width 0.8) (layer F.Cu) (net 7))
 (segment (start 200.875 93.25) (end 200.19571 93.92929) (width 0.8) (layer F.Cu) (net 7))
 (segment (start 199.5 95.975) (end 199.5 95) (width 1.1) (layer F.Cu) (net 7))
 (segment (start 199.5 96) (end 199.5 95.975) (width 1.1) (layer F.Cu) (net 7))
 (segment (start 200 96.5) (end 199.5 96) (width 1.1) (layer F.Cu) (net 7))
 (segment (start 200 97.58) (end 200 96.5) (width 1.1) (layer F.Cu) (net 7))
 (segment (start 198.58 99) (end 200 97.58) (width 1.1) (layer F.Cu) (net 7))
 (segment (start 195.100001 97.399999) (end 193.5 99) (width 1.1) (layer B.Cu) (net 7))
 (segment (start 196.979999 97.399999) (end 195.100001 97.399999) (width 1.1) (layer B.Cu) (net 7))
 (segment (start 198.58 99) (end 196.979999 97.399999) (width 1.1) (layer B.Cu) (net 7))
 (segment (start 190.6 95.5) (end 192.35 97.25) (width 1.1) (layer F.Cu) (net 9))
 (segment (start 189.25 95.5) (end 190.6 95.5) (width 1.1) (layer F.Cu) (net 9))
 (segment (start 196.04 97.797919) (end 196.04 99) (width 1.1) (layer F.Cu) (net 9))
 (segment (start 195.492081 97.25) (end 196.04 97.797919) (width 1.1) (layer F.Cu) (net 9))
 (segment (start 192.35 97.25) (end 195.492081 97.25) (width 1.1) (layer F.Cu) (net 9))
 (segment (start 170.32929 99.12929) (end 170.85 99.65) (width 0.25) (layer F.Cu) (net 11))
 (segment (start 153 99.575) (end 153.461612 99.113388) (width 0.25) (layer F.Cu) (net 11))
 (segment (start 168.62499 97.42499) (end 170.32929 99.12929) (width 0.25) (layer F.Cu) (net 11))
 (segment (start 153.461612 99.113388) (end 154.886612 99.113388) (width 0.25) (layer F.Cu) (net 11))
 (segment (start 154.886612 99.113388) (end 155.5 98.5) (width 0.25) (layer F.Cu) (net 11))
 (segment (start 158.151456 98.5) (end 159.226466 97.42499) (width 0.25) (layer F.Cu) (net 11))
 (segment (start 155.5 98.5) (end 158.151456 98.5) (width 0.25) (layer F.Cu) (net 11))
 (segment (start 159.226466 97.42499) (end 168.62499 97.42499) (width 0.25) (layer F.Cu) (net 11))
 (segment (start 171.75 100.85) (end 171.97501 100.62499) (width 0.25) (layer F.Cu) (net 3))
 (segment (start 173.25 89.5) (end 173.754682 89.5) (width 0.25) (layer F.Cu) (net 3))
 (segment (start 173.779692 89.47499) (end 175.290008 89.47499) (width 0.25) (layer F.Cu) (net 3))
 (segment (start 168.527834 95.75) (end 168.527834 94.75483) (width 0.25) (layer F.Cu) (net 3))
 (segment (start 173 89.75) (end 173.25 89.5) (width 0.25) (layer F.Cu) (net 3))
 (segment (start 168.527834 94.75483) (end 168.1 94.326996) (width 0.25) (layer F.Cu) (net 3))
 (segment (start 173.754682 89.5) (end 173.779692 89.47499) (width 0.25) (layer F.Cu) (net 3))
 (segment (start 171.97501 99.197176) (end 168.527834 95.75) (width 0.25) (layer F.Cu) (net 3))
 (segment (start 171.97501 100.62499) (end 171.97501 99.197176) (width 0.25) (layer F.Cu) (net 3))
 (segment (start 177.660001 89.424999) (end 177.709992 89.47499) (width 0.25) (layer F.Cu) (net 3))
 (segment (start 170.85 100.85) (end 171.75 100.85) (width 0.25) (layer F.Cu) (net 3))
 (segment (start 168.1 94.326996) (end 168.1 89.95) (width 0.25) (layer F.Cu) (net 3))
 (segment (start 168.3 89.75) (end 173 89.75) (width 0.25) (layer F.Cu) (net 3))
 (segment (start 168.1 89.95) (end 168.3 89.75) (width 0.25) (layer F.Cu) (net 3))
 (segment (start 175.290008 89.47499) (end 175.339999 89.424999) (width 0.25) (layer F.Cu) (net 3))
 (segment (start 175.339999 89.424999) (end 177.660001 89.424999) (width 0.25) (layer F.Cu) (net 3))
 (segment (start 183.9 89.59998) (end 183.77501 89.47499) (width 0.25) (layer F.Cu) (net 3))
 (segment (start 183.9 91.025) (end 183.9 89.59998) (width 0.25) (layer F.Cu) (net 3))
 (segment (start 177.709992 89.47499) (end 183.77501 89.47499) (width 0.25) (layer F.Cu) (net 3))
 (segment (start 201.25 90.925) (end 201.15 91.025) (width 0.25) (layer F.Cu) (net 3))
 (segment (start 201.25 90.25) (end 201.25 90.925) (width 0.25) (layer F.Cu) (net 3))
 (segment (start 199.924999 88.924999) (end 201.25 90.25) (width 0.25) (layer F.Cu) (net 3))
 (segment (start 189.994981 88.924999) (end 199.924999 88.924999) (width 0.25) (layer F.Cu) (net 3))
 (segment (start 183.77501 89.47499) (end 189.44499 89.47499) (width 0.25) (layer F.Cu) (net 3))
 (segment (start 189.44499 89.47499) (end 189.994981 88.924999) (width 0.25) (layer F.Cu) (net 3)))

